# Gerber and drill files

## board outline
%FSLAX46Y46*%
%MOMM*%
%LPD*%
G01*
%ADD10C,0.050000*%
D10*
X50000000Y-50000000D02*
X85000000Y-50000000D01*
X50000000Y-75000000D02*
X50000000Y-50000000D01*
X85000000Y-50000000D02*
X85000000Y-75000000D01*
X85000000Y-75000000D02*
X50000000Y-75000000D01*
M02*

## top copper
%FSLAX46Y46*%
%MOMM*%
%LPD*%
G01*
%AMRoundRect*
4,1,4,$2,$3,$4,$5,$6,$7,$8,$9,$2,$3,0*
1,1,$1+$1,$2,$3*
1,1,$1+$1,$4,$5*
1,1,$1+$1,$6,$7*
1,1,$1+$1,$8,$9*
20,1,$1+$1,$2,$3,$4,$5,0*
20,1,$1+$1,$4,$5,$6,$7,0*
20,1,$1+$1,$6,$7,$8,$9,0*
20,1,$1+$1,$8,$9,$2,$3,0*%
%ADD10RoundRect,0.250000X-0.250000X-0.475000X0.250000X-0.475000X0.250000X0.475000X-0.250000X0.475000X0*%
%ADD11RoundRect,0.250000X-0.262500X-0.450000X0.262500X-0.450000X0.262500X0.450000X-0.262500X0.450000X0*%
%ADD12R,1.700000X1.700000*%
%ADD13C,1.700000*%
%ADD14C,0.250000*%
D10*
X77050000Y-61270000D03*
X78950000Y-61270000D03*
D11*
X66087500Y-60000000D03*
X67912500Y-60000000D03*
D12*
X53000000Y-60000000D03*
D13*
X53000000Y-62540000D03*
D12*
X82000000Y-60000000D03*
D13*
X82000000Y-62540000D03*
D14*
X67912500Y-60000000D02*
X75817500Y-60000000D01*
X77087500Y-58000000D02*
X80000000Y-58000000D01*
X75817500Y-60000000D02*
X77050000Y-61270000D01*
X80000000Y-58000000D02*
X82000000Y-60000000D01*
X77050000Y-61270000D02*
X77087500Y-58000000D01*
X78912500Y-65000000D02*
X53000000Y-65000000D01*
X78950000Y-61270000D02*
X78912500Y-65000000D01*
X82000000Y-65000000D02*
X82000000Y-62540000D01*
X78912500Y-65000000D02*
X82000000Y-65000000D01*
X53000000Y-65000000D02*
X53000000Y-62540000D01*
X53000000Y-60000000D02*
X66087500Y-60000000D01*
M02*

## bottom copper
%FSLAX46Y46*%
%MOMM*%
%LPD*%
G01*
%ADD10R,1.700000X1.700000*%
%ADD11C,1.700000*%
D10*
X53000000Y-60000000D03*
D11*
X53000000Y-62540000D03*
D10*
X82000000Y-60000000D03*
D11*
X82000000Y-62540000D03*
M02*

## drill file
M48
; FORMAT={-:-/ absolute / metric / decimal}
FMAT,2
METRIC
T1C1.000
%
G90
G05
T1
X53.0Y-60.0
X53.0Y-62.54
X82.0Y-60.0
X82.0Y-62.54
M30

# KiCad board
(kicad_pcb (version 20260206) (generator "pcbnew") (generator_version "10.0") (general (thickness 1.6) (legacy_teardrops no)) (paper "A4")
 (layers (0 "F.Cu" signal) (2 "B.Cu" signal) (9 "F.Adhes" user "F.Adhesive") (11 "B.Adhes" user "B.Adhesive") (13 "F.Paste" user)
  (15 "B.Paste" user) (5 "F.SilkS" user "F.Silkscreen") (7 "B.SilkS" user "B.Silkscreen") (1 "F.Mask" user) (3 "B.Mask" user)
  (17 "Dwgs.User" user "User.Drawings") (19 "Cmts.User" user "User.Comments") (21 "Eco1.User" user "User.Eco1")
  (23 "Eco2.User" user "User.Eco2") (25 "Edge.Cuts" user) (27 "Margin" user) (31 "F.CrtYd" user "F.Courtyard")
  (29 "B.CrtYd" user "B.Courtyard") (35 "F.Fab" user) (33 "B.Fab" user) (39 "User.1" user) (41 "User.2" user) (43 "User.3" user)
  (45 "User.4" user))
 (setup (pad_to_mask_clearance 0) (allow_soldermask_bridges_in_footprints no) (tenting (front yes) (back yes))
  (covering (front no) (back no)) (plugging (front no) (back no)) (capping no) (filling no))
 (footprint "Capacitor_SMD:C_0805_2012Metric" (layer "F.Cu") (at 78 61.27)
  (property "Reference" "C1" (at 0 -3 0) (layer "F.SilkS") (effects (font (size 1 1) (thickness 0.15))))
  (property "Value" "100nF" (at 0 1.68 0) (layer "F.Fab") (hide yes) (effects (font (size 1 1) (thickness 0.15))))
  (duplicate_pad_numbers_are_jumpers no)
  (pad "1" smd roundrect (at -0.95 0) (size 1 1.45) (layers "F.Cu" "F.Mask" "F.Paste") (roundrect_rratio 0.25) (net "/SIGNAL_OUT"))
  (pad "2" smd roundrect (at 0.95 0) (size 1 1.45) (layers "F.Cu" "F.Mask" "F.Paste") (roundrect_rratio 0.25) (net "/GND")))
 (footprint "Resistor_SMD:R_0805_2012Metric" (layer "F.Cu") (at 67 60)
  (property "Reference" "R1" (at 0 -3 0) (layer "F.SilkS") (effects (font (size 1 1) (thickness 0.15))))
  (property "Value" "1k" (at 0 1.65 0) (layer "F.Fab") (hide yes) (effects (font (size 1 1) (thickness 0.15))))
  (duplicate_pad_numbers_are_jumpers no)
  (pad "1" smd roundrect (at -0.9125 0) (size 1.025 1.4) (layers "F.Cu" "F.Mask" "F.Paste") (roundrect_rratio 0.243902) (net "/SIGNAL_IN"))
  (pad "2" smd roundrect (at 0.9125 0) (size 1.025 1.4) (layers "F.Cu" "F.Mask" "F.Paste") (roundrect_rratio 0.243902) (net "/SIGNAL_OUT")))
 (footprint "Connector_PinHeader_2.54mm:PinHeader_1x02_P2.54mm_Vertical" (layer "F.Cu") (at 53 60)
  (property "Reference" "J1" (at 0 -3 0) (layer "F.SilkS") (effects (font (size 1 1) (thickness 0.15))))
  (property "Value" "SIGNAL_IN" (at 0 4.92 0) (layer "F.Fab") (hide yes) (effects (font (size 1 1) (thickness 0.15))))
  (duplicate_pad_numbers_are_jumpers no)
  (pad "1" thru_hole rect (at 0 0) (size 1.7 1.7) (drill 1) (layers "*.Cu" "*.Mask") (remove_unused_layers no) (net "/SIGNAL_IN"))
  (pad "2" thru_hole circle (at 0 2.54) (size 1.7 1.7) (drill 1) (layers "*.Cu" "*.Mask") (remove_unused_layers no) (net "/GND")))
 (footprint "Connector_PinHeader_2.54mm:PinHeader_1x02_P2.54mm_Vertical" (layer "F.Cu") (at 82 60)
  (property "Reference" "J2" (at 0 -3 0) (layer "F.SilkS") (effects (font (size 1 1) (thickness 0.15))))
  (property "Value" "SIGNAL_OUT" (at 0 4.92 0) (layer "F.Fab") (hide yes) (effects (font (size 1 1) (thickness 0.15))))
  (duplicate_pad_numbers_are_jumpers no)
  (pad "1" thru_hole rect (at 0 0) (size 1.7 1.7) (drill 1) (layers "*.Cu" "*.Mask") (remove_unused_layers no) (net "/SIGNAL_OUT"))
  (pad "2" thru_hole circle (at 0 2.54) (size 1.7 1.7) (drill 1) (layers "*.Cu" "*.Mask") (remove_unused_layers no) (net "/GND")))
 (gr_line (start 50 50) (end 85 50) (stroke (width 0.05) (type default)) (layer "Edge.Cuts"))
 (gr_line (start 50 75) (end 50 50) (stroke (width 0.05) (type default)) (layer "Edge.Cuts"))
 (gr_line (start 85 50) (end 85 75) (stroke (width 0.05) (type default)) (layer "Edge.Cuts"))
 (gr_line (start 85 75) (end 50 75) (stroke (width 0.05) (type default)) (layer "Edge.Cuts"))
 (segment (start 67.9125 60) (end 75.8175 60) (width 0.25) (layer "F.Cu") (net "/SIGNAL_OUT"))
 (segment (start 77.0875 58) (end 80 58) (width 0.25) (layer "F.Cu") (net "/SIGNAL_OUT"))
 (segment (start 75.8175 60) (end 77.05 61.27) (width 0.25) (layer "F.Cu") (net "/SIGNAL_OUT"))
 (segment (start 80 58) (end 82 60) (width 0.25) (layer "F.Cu") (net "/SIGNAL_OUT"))
 (segment (start 77.05 61.27) (end 77.0875 58) (width 0.25) (layer "F.Cu") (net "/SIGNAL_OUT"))
 (segment (start 78.9125 65) (end 53 65) (width 0.25) (layer "F.Cu") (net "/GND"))
 (segment (start 78.95 61.27) (end 78.9125 65) (width 0.25) (layer "F.Cu") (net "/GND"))
 (segment (start 82 65) (end 82 62.54) (width 0.25) (layer "F.Cu") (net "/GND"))
 (segment (start 78.9125 65) (end 82 65) (width 0.25) (layer "F.Cu") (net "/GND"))
 (segment (start 53 65) (end 53 62.54) (width 0.25) (layer "F.Cu") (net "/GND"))
 (segment (start 53 60) (end 66.0875 60) (width 0.25) (layer "F.Cu") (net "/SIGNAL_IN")))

